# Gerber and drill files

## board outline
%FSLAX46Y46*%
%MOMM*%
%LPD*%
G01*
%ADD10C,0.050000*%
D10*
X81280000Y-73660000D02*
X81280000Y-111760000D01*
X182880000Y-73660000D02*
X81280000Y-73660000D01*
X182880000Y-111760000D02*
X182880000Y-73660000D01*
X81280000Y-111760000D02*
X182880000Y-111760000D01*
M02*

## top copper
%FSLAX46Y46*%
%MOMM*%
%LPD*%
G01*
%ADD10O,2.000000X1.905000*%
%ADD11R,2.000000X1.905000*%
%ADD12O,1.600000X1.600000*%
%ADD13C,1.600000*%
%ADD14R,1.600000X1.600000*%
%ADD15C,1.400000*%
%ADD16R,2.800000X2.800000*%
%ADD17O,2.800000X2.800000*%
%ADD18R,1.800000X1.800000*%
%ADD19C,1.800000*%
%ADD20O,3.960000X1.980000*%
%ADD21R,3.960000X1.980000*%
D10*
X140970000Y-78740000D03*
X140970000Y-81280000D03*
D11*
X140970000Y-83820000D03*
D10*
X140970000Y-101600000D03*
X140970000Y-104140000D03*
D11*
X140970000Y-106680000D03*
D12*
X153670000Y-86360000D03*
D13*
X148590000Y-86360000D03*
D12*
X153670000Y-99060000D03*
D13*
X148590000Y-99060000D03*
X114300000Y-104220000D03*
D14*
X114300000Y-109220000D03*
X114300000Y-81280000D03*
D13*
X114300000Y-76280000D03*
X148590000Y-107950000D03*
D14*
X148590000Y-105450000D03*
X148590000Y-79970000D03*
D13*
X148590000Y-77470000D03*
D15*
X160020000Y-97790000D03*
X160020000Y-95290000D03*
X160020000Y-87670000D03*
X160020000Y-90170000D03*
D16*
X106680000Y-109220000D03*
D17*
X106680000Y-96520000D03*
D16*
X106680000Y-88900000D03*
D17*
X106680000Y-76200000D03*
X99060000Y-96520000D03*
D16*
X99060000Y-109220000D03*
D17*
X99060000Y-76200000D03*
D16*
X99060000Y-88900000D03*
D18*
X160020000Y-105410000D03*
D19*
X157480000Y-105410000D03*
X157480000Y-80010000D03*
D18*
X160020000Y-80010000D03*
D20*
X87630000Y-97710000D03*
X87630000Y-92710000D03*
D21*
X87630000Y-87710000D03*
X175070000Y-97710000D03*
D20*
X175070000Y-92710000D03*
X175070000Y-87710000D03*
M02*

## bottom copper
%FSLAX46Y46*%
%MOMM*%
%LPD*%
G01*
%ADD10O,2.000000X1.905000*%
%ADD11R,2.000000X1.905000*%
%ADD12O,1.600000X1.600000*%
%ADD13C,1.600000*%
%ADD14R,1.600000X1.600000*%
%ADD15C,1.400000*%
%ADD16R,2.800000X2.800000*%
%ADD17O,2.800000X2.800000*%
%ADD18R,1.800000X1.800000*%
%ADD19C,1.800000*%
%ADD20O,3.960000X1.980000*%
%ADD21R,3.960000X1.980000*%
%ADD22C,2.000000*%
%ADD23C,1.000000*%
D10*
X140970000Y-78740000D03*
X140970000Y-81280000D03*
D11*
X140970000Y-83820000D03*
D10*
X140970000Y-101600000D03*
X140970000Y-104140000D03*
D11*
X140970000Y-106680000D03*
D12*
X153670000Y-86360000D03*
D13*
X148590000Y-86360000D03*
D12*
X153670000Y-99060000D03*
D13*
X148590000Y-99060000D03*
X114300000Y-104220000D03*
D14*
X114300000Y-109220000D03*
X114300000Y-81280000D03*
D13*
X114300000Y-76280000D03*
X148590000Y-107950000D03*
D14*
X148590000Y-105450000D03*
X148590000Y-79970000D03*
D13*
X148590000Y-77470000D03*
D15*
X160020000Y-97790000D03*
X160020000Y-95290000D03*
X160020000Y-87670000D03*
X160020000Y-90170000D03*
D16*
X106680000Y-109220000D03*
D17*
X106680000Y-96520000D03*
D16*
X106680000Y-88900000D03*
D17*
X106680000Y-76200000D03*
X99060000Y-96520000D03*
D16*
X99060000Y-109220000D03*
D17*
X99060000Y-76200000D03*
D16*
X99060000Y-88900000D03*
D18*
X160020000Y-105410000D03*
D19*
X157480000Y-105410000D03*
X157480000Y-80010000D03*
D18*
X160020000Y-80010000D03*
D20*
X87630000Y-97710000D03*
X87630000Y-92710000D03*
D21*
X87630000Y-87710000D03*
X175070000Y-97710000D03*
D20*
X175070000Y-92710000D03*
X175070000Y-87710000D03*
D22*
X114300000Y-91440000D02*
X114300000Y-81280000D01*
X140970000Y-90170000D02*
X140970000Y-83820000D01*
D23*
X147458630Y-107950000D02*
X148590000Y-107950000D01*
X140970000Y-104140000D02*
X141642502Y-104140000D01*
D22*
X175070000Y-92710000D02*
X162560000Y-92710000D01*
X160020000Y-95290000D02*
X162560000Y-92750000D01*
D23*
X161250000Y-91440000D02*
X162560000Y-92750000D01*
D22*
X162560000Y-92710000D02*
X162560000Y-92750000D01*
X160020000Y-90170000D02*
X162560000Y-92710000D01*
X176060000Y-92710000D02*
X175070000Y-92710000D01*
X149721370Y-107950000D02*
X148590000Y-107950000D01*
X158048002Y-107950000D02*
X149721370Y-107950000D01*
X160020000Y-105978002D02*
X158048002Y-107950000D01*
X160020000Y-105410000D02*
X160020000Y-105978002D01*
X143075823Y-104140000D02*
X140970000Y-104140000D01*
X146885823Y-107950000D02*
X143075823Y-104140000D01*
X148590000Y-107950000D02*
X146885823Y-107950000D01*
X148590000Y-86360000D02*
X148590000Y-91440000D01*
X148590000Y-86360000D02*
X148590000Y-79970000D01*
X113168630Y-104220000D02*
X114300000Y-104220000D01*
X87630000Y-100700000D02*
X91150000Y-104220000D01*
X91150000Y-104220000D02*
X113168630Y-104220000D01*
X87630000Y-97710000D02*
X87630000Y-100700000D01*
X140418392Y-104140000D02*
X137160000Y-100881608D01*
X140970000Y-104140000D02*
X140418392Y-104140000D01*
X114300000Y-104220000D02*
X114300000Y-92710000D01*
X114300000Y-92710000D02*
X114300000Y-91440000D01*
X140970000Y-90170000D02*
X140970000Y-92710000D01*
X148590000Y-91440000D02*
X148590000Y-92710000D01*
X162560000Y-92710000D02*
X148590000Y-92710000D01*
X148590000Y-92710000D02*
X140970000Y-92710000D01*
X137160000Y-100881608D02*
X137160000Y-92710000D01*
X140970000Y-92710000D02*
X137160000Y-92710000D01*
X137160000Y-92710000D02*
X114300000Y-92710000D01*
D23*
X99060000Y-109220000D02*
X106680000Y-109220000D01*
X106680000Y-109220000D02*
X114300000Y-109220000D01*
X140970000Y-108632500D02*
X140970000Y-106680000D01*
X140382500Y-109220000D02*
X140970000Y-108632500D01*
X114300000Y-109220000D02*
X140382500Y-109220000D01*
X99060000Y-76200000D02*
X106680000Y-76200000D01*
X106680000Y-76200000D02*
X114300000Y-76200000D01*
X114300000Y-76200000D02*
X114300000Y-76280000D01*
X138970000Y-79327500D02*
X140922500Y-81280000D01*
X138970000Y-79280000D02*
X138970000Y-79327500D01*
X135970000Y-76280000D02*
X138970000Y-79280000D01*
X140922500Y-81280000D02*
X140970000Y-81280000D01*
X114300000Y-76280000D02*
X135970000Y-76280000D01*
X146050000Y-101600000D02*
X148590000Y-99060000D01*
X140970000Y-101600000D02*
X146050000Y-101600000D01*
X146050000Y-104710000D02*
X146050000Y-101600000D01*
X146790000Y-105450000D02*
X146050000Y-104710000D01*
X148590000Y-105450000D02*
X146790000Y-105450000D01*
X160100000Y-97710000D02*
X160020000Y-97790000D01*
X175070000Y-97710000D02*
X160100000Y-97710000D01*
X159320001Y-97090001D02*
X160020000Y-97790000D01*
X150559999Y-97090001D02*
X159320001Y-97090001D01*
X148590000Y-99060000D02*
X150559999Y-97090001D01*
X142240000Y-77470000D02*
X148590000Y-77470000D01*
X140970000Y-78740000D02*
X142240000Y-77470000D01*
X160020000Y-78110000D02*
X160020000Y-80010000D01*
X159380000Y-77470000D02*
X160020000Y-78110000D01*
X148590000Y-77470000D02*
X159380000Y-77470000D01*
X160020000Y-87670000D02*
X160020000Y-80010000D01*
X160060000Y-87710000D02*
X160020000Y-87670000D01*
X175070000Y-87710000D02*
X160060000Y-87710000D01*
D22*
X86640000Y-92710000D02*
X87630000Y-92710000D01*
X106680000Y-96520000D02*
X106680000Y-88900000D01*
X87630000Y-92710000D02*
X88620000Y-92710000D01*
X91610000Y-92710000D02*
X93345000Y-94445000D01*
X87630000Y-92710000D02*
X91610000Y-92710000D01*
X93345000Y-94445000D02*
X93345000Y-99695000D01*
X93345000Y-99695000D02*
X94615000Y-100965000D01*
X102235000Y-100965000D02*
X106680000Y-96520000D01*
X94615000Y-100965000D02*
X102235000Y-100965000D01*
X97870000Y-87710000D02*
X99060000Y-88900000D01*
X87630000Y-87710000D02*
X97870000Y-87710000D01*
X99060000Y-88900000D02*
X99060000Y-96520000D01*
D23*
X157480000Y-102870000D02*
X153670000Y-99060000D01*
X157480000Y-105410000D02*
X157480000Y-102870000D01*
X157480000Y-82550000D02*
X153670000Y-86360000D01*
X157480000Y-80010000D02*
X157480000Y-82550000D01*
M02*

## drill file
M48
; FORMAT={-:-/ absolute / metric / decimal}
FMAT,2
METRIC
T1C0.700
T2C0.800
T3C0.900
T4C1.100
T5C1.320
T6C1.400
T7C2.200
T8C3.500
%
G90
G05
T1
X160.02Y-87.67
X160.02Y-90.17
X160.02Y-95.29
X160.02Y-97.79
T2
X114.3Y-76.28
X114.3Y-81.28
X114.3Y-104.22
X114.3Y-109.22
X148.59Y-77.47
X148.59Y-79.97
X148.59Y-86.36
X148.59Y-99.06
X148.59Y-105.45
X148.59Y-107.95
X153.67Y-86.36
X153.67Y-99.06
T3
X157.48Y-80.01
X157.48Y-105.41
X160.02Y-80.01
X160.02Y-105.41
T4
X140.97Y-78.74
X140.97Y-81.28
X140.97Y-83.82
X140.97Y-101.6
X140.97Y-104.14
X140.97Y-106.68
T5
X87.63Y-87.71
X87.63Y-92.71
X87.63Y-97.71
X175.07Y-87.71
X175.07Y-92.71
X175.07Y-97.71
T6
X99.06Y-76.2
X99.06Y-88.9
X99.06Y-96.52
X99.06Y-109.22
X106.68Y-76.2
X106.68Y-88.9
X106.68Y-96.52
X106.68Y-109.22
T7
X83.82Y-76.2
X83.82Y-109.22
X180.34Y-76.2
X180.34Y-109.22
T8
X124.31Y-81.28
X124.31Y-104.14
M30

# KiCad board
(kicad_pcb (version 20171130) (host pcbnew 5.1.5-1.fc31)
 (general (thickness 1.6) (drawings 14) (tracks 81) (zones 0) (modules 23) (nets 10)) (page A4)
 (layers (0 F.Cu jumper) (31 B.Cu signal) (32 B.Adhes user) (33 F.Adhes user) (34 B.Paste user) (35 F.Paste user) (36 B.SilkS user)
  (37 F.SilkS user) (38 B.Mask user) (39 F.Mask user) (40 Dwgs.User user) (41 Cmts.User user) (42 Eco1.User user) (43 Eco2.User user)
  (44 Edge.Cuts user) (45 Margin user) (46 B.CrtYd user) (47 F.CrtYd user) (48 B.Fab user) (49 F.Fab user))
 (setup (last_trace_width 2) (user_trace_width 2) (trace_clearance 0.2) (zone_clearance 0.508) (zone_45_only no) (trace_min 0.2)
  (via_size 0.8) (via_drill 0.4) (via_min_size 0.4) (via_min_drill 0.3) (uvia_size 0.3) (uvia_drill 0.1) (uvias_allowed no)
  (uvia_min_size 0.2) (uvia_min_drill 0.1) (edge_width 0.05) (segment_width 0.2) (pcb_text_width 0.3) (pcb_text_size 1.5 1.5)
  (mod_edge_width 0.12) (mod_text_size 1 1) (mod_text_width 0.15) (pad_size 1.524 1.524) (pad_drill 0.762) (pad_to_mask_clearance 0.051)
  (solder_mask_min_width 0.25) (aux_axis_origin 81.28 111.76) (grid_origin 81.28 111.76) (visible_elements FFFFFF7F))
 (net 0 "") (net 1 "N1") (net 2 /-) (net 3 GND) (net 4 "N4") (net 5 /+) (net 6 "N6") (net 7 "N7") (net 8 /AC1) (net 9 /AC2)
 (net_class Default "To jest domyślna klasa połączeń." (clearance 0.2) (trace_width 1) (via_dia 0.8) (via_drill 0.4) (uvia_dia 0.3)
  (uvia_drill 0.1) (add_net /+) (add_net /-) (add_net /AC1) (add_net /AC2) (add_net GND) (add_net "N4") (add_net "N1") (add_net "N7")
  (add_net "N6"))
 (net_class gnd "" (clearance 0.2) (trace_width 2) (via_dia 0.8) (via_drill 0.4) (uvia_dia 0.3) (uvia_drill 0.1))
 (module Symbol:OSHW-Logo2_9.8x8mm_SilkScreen (layer F.Cu) (at 114.3 87.63)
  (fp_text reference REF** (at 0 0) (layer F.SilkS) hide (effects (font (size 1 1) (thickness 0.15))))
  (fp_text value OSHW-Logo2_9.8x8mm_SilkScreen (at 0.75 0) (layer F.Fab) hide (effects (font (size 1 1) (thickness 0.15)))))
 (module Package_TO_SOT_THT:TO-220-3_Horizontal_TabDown (layer F.Cu) (at 140.97 83.82 90)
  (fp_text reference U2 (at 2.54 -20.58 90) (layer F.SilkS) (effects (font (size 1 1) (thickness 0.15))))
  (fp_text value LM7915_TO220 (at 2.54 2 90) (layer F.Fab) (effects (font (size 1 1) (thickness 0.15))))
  (pad 3 thru_hole oval (at 5.08 0 90) (size 1.905 2) (drill 1.1) (layers *.Cu *.Mask) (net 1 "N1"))
  (pad 2 thru_hole oval (at 2.54 0 90) (size 1.905 2) (drill 1.1) (layers *.Cu *.Mask) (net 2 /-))
  (pad 1 thru_hole rect (at 0 0 90) (size 1.905 2) (drill 1.1) (layers *.Cu *.Mask) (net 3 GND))
  (pad "" np_thru_hole oval (at 2.54 -16.66 90) (size 3.5 3.5) (drill 3.5) (layers *.Cu *.Mask)))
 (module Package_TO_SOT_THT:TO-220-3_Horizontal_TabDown (layer F.Cu) (at 140.97 106.68 90)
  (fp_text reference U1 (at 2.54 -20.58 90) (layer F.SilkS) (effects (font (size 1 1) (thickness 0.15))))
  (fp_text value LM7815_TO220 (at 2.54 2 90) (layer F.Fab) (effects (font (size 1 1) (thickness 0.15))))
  (pad 3 thru_hole oval (at 5.08 0 90) (size 1.905 2) (drill 1.1) (layers *.Cu *.Mask) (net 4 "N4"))
  (pad 2 thru_hole oval (at 2.54 0 90) (size 1.905 2) (drill 1.1) (layers *.Cu *.Mask) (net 3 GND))
  (pad 1 thru_hole rect (at 0 0 90) (size 1.905 2) (drill 1.1) (layers *.Cu *.Mask) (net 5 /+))
  (pad "" np_thru_hole oval (at 2.54 -16.66 90) (size 3.5 3.5) (drill 3.5) (layers *.Cu *.Mask)))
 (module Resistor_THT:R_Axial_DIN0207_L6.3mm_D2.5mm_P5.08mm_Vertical (layer F.Cu) (at 148.59 86.36)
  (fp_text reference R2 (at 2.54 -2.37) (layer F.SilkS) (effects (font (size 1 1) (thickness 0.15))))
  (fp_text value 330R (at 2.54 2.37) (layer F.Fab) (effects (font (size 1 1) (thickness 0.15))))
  (pad 2 thru_hole oval (at 5.08 0) (size 1.6 1.6) (drill 0.8) (layers *.Cu *.Mask) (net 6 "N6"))
  (pad 1 thru_hole circle (at 0 0) (size 1.6 1.6) (drill 0.8) (layers *.Cu *.Mask) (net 3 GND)))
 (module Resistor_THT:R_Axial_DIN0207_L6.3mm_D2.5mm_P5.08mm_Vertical (layer F.Cu) (at 148.59 99.06)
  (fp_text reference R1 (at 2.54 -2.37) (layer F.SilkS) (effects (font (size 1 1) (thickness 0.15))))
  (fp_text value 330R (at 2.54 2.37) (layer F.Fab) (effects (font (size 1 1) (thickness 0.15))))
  (pad 2 thru_hole oval (at 5.08 0) (size 1.6 1.6) (drill 0.8) (layers *.Cu *.Mask) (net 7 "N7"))
  (pad 1 thru_hole circle (at 0 0) (size 1.6 1.6) (drill 0.8) (layers *.Cu *.Mask) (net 4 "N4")))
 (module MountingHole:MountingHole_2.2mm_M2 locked (layer F.Cu) (at 83.82 109.22)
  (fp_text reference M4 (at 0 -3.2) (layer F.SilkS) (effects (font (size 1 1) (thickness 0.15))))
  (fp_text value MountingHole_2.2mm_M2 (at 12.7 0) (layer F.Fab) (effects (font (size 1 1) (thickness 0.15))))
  (pad 1 np_thru_hole circle (at 0 0) (size 2.2 2.2) (drill 2.2) (layers *.Cu *.Mask)))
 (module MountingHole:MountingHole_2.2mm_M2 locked (layer F.Cu) (at 180.34 109.22)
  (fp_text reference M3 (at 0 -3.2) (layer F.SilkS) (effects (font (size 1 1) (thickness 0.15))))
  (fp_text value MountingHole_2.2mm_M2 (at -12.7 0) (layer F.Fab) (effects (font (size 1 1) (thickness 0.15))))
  (pad 1 np_thru_hole circle (at 0 0) (size 2.2 2.2) (drill 2.2) (layers *.Cu *.Mask)))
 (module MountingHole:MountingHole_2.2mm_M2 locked (layer F.Cu) (at 180.34 76.2)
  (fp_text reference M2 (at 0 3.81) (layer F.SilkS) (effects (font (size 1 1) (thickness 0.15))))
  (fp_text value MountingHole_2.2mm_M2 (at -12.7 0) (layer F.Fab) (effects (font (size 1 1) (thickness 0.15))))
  (pad 1 np_thru_hole circle (at 0 0) (size 2.2 2.2) (drill 2.2) (layers *.Cu *.Mask)))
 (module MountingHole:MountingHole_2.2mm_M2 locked (layer F.Cu) (at 83.82 76.2)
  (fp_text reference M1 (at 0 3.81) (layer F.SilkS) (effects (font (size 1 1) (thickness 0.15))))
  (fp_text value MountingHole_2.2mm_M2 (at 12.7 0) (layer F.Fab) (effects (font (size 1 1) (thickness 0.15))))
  (pad 1 np_thru_hole circle (at 0 0) (size 2.2 2.2) (drill 2.2) (layers *.Cu *.Mask)))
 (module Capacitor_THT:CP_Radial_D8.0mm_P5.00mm (layer F.Cu) (at 114.3 109.22 90)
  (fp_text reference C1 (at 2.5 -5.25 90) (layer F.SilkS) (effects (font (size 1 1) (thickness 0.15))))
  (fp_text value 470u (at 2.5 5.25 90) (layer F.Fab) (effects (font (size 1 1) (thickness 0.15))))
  (pad 2 thru_hole circle (at 5 0 90) (size 1.6 1.6) (drill 0.8) (layers *.Cu *.Mask) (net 3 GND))
  (pad 1 thru_hole rect (at 0 0 90) (size 1.6 1.6) (drill 0.8) (layers *.Cu *.Mask) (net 5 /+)))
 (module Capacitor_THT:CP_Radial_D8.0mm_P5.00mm (layer F.Cu) (at 114.3 81.28 90)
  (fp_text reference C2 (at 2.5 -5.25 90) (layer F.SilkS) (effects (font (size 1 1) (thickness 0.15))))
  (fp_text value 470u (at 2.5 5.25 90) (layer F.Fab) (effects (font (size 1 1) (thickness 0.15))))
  (pad 1 thru_hole rect (at 0 0 90) (size 1.6 1.6) (drill 0.8) (layers *.Cu *.Mask) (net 3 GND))
  (pad 2 thru_hole circle (at 5 0 90) (size 1.6 1.6) (drill 0.8) (layers *.Cu *.Mask) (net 2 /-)))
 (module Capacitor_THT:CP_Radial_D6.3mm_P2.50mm (layer F.Cu) (at 148.59 105.45 270)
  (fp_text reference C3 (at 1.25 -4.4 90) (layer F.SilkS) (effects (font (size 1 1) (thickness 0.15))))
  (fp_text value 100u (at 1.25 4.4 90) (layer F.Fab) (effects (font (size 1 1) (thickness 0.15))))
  (pad 2 thru_hole circle (at 2.5 0 270) (size 1.6 1.6) (drill 0.8) (layers *.Cu *.Mask) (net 3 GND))
  (pad 1 thru_hole rect (at 0 0 270) (size 1.6 1.6) (drill 0.8) (layers *.Cu *.Mask) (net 4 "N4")))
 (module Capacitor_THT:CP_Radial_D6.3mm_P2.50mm (layer F.Cu) (at 148.59 79.97 90)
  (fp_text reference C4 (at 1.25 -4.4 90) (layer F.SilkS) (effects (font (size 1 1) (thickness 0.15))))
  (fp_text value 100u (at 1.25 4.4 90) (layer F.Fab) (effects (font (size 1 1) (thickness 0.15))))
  (pad 1 thru_hole rect (at 0 0 90) (size 1.6 1.6) (drill 0.8) (layers *.Cu *.Mask) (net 3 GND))
  (pad 2 thru_hole circle (at 2.5 0 90) (size 1.6 1.6) (drill 0.8) (layers *.Cu *.Mask) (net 1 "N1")))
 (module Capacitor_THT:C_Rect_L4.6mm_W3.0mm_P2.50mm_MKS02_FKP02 (layer F.Cu) (at 160.02 97.79 90)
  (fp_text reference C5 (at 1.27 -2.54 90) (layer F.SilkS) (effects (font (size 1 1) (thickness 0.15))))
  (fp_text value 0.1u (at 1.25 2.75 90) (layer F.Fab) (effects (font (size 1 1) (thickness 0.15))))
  (pad 1 thru_hole circle (at 0 0 90) (size 1.4 1.4) (drill 0.7) (layers *.Cu *.Mask) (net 4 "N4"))
  (pad 2 thru_hole circle (at 2.5 0 90) (size 1.4 1.4) (drill 0.7) (layers *.Cu *.Mask) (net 3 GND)))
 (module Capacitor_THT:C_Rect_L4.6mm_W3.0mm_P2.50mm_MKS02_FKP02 (layer F.Cu) (at 160.02 90.17 90)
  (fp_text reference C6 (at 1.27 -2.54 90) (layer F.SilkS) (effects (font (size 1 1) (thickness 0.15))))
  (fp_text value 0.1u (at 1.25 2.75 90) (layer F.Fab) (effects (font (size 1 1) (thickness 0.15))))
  (pad 2 thru_hole circle (at 2.5 0 90) (size 1.4 1.4) (drill 0.7) (layers *.Cu *.Mask) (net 1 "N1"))
  (pad 1 thru_hole circle (at 0 0 90) (size 1.4 1.4) (drill 0.7) (layers *.Cu *.Mask) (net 3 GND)))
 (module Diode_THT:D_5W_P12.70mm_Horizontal (layer F.Cu) (at 106.68 109.22 90)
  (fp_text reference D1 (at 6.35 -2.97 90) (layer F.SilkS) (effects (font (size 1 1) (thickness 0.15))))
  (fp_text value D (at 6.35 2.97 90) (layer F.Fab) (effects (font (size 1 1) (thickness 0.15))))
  (pad 1 thru_hole rect (at 0 0 90) (size 2.8 2.8) (drill 1.4) (layers *.Cu *.Mask) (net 5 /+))
  (pad 2 thru_hole oval (at 12.7 0 90) (size 2.8 2.8) (drill 1.4) (layers *.Cu *.Mask) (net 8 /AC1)))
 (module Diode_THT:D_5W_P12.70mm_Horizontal (layer F.Cu) (at 106.68 88.9 90)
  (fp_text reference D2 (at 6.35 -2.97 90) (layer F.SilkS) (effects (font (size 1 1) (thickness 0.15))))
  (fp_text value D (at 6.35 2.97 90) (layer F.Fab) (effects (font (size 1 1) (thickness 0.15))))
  (pad 1 thru_hole rect (at 0 0 90) (size 2.8 2.8) (drill 1.4) (layers *.Cu *.Mask) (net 8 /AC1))
  (pad 2 thru_hole oval (at 12.7 0 90) (size 2.8 2.8) (drill 1.4) (layers *.Cu *.Mask) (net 2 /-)))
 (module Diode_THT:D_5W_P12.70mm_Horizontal (layer F.Cu) (at 99.06 109.22 90)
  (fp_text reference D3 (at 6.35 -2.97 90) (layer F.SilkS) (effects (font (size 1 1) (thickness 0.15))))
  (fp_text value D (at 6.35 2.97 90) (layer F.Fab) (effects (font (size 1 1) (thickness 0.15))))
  (pad 2 thru_hole oval (at 12.7 0 90) (size 2.8 2.8) (drill 1.4) (layers *.Cu *.Mask) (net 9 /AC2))
  (pad 1 thru_hole rect (at 0 0 90) (size 2.8 2.8) (drill 1.4) (layers *.Cu *.Mask) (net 5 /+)))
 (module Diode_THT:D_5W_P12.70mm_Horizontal (layer F.Cu) (at 99.06 88.9 90)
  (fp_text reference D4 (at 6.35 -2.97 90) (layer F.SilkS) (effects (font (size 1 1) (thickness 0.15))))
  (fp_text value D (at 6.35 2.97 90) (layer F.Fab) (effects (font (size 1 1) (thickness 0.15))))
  (pad 2 thru_hole oval (at 12.7 0 90) (size 2.8 2.8) (drill 1.4) (layers *.Cu *.Mask) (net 2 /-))
  (pad 1 thru_hole rect (at 0 0 90) (size 2.8 2.8) (drill 1.4) (layers *.Cu *.Mask) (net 9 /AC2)))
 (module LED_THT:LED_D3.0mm (layer F.Cu) (at 160.02 105.41 180)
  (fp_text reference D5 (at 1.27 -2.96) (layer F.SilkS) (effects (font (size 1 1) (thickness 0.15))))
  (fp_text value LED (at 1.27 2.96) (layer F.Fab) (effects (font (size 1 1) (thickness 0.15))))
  (pad 1 thru_hole rect (at 0 0 180) (size 1.8 1.8) (drill 0.9) (layers *.Cu *.Mask) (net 3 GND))
  (pad 2 thru_hole circle (at 2.54 0 180) (size 1.8 1.8) (drill 0.9) (layers *.Cu *.Mask) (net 7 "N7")))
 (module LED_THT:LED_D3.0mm (layer F.Cu) (at 160.02 80.01 180)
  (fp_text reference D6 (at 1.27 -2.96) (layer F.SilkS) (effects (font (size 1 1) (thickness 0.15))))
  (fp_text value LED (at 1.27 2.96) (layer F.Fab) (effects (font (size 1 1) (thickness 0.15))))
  (pad 2 thru_hole circle (at 2.54 0 180) (size 1.8 1.8) (drill 0.9) (layers *.Cu *.Mask) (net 6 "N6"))
  (pad 1 thru_hole rect (at 0 0 180) (size 1.8 1.8) (drill 0.9) (layers *.Cu *.Mask) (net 1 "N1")))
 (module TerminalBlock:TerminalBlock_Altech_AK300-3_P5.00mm (layer F.Cu) (at 87.63 87.71 270)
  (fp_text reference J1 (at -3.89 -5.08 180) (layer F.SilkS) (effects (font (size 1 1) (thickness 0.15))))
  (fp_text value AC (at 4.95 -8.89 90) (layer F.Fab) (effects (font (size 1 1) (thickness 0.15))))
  (pad 3 thru_hole oval (at 10 0 270) (size 1.98 3.96) (drill 1.32) (layers *.Cu *.Mask) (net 3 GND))
  (pad 2 thru_hole oval (at 5 0 270) (size 1.98 3.96) (drill 1.32) (layers *.Cu *.Mask) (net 8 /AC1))
  (pad 1 thru_hole rect (at 0 0 270) (size 1.98 3.96) (drill 1.32) (layers *.Cu *.Mask) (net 9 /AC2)))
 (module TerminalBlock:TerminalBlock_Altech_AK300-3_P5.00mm (layer F.Cu) (at 175.07 97.71 90)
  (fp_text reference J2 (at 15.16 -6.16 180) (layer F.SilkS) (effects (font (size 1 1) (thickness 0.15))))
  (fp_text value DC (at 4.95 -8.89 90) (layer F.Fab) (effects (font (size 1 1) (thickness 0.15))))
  (pad 1 thru_hole rect (at 0 0 90) (size 1.98 3.96) (drill 1.32) (layers *.Cu *.Mask) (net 4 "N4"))
  (pad 2 thru_hole oval (at 5 0 90) (size 1.98 3.96) (drill 1.32) (layers *.Cu *.Mask) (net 3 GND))
  (pad 3 thru_hole oval (at 10 0 90) (size 1.98 3.96) (drill 1.32) (layers *.Cu *.Mask) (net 1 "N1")))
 (gr_line (start 81.28 73.66) (end 81.28 111.76) (layer Edge.Cuts) (width 0.05))
 (gr_line (start 182.88 73.66) (end 81.28 73.66) (layer Edge.Cuts) (width 0.05))
 (gr_line (start 182.88 111.76) (end 182.88 73.66) (layer Edge.Cuts) (width 0.05))
 (gr_line (start 81.28 111.76) (end 182.88 111.76) (layer Edge.Cuts) (width 0.05))
 (segment (start 114.3 91.44) (end 114.3 81.28) (width 2) (layer B.Cu) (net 3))
 (segment (start 140.97 90.17) (end 140.97 83.82) (width 2) (layer B.Cu) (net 3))
 (segment (start 147.45863 107.95) (end 148.59 107.95) (width 1) (layer B.Cu) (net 3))
 (segment (start 140.97 104.14) (end 141.642502 104.14) (width 1) (layer B.Cu) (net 3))
 (segment (start 175.07 92.71) (end 162.56 92.71) (width 2) (layer B.Cu) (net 3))
 (segment (start 160.02 95.29) (end 162.56 92.75) (width 2) (layer B.Cu) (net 3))
 (segment (start 161.25 91.44) (end 162.56 92.75) (width 1) (layer B.Cu) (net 3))
 (segment (start 162.56 92.71) (end 162.56 92.75) (width 2) (layer B.Cu) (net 3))
 (segment (start 160.02 90.17) (end 162.56 92.71) (width 2) (layer B.Cu) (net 3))
 (segment (start 176.06 92.71) (end 175.07 92.71) (width 2) (layer B.Cu) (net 3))
 (segment (start 149.72137 107.95) (end 148.59 107.95) (width 2) (layer B.Cu) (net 3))
 (segment (start 158.048002 107.95) (end 149.72137 107.95) (width 2) (layer B.Cu) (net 3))
 (segment (start 160.02 105.978002) (end 158.048002 107.95) (width 2) (layer B.Cu) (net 3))
 (segment (start 160.02 105.41) (end 160.02 105.978002) (width 2) (layer B.Cu) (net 3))
 (segment (start 143.075823 104.14) (end 140.97 104.14) (width 2) (layer B.Cu) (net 3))
 (segment (start 146.885823 107.95) (end 143.075823 104.14) (width 2) (layer B.Cu) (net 3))
 (segment (start 148.59 107.95) (end 146.885823 107.95) (width 2) (layer B.Cu) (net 3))
 (segment (start 148.59 86.36) (end 148.59 91.44) (width 2) (layer B.Cu) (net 3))
 (segment (start 148.59 86.36) (end 148.59 79.97) (width 2) (layer B.Cu) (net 3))
 (segment (start 113.16863 104.22) (end 114.3 104.22) (width 2) (layer B.Cu) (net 3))
 (segment (start 87.63 100.7) (end 91.15 104.22) (width 2) (layer B.Cu) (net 3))
 (segment (start 91.15 104.22) (end 113.16863 104.22) (width 2) (layer B.Cu) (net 3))
 (segment (start 87.63 97.71) (end 87.63 100.7) (width 2) (layer B.Cu) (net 3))
 (segment (start 140.418392 104.14) (end 137.16 100.881608) (width 2) (layer B.Cu) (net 3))
 (segment (start 140.97 104.14) (end 140.418392 104.14) (width 2) (layer B.Cu) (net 3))
 (segment (start 114.3 104.22) (end 114.3 92.71) (width 2) (layer B.Cu) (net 3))
 (segment (start 114.3 92.71) (end 114.3 91.44) (width 2) (layer B.Cu) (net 3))
 (segment (start 140.97 90.17) (end 140.97 92.71) (width 2) (layer B.Cu) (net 3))
 (segment (start 148.59 91.44) (end 148.59 92.71) (width 2) (layer B.Cu) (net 3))
 (segment (start 162.56 92.71) (end 148.59 92.71) (width 2) (layer B.Cu) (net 3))
 (segment (start 148.59 92.71) (end 140.97 92.71) (width 2) (layer B.Cu) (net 3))
 (segment (start 137.16 100.881608) (end 137.16 92.71) (width 2) (layer B.Cu) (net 3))
 (segment (start 140.97 92.71) (end 137.16 92.71) (width 2) (layer B.Cu) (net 3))
 (segment (start 137.16 92.71) (end 114.3 92.71) (width 2) (layer B.Cu) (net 3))
 (segment (start 99.06 109.22) (end 106.68 109.22) (width 1) (layer B.Cu) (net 5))
 (segment (start 106.68 109.22) (end 114.3 109.22) (width 1) (layer B.Cu) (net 5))
 (segment (start 140.97 108.6325) (end 140.97 106.68) (width 1) (layer B.Cu) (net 5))
 (segment (start 140.3825 109.22) (end 140.97 108.6325) (width 1) (layer B.Cu) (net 5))
 (segment (start 114.3 109.22) (end 140.3825 109.22) (width 1) (layer B.Cu) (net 5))
 (segment (start 99.06 76.2) (end 106.68 76.2) (width 1) (layer B.Cu) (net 2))
 (segment (start 106.68 76.2) (end 114.3 76.2) (width 1) (layer B.Cu) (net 2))
 (segment (start 114.3 76.2) (end 114.3 76.28) (width 1) (layer B.Cu) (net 2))
 (segment (start 138.97 79.3275) (end 140.9225 81.28) (width 1) (layer B.Cu) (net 2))
 (segment (start 138.97 79.28) (end 138.97 79.3275) (width 1) (layer B.Cu) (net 2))
 (segment (start 135.97 76.28) (end 138.97 79.28) (width 1) (layer B.Cu) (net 2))
 (segment (start 140.9225 81.28) (end 140.97 81.28) (width 1) (layer B.Cu) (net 2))
 (segment (start 114.3 76.28) (end 135.97 76.28) (width 1) (layer B.Cu) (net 2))
 (segment (start 146.05 101.6) (end 148.59 99.06) (width 1) (layer B.Cu) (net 4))
 (segment (start 140.97 101.6) (end 146.05 101.6) (width 1) (layer B.Cu) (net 4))
 (segment (start 146.05 104.71) (end 146.05 101.6) (width 1) (layer B.Cu) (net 4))
 (segment (start 146.79 105.45) (end 146.05 104.71) (width 1) (layer B.Cu) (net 4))
 (segment (start 148.59 105.45) (end 146.79 105.45) (width 1) (layer B.Cu) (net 4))
 (segment (start 160.1 97.71) (end 160.02 97.79) (width 1) (layer B.Cu) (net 4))
 (segment (start 175.07 97.71) (end 160.1 97.71) (width 1) (layer B.Cu) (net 4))
 (segment (start 159.320001 97.090001) (end 160.02 97.79) (width 1) (layer B.Cu) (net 4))
 (segment (start 150.559999 97.090001) (end 159.320001 97.090001) (width 1) (layer B.Cu) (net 4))
 (segment (start 148.59 99.06) (end 150.559999 97.090001) (width 1) (layer B.Cu) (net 4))
 (segment (start 142.24 77.47) (end 148.59 77.47) (width 1) (layer B.Cu) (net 1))
 (segment (start 140.97 78.74) (end 142.24 77.47) (width 1) (layer B.Cu) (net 1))
 (segment (start 160.02 78.11) (end 160.02 80.01) (width 1) (layer B.Cu) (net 1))
 (segment (start 159.38 77.47) (end 160.02 78.11) (width 1) (layer B.Cu) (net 1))
 (segment (start 148.59 77.47) (end 159.38 77.47) (width 1) (layer B.Cu) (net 1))
 (segment (start 160.02 87.67) (end 160.02 80.01) (width 1) (layer B.Cu) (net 1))
 (segment (start 160.06 87.71) (end 160.02 87.67) (width 1) (layer B.Cu) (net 1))
 (segment (start 175.07 87.71) (end 160.06 87.71) (width 1) (layer B.Cu) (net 1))
 (segment (start 86.64 92.71) (end 87.63 92.71) (width 2) (layer B.Cu) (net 8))
 (segment (start 106.68 96.52) (end 106.68 88.9) (width 2) (layer B.Cu) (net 8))
 (segment (start 87.63 92.71) (end 88.62 92.71) (width 2) (layer B.Cu) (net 8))
 (segment (start 91.61 92.71) (end 93.345 94.445) (width 2) (layer B.Cu) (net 8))
 (segment (start 87.63 92.71) (end 91.61 92.71) (width 2) (layer B.Cu) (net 8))
 (segment (start 93.345 94.445) (end 93.345 99.695) (width 2) (layer B.Cu) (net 8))
 (segment (start 93.345 99.695) (end 94.615 100.965) (width 2) (layer B.Cu) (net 8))
 (segment (start 102.235 100.965) (end 106.68 96.52) (width 2) (layer B.Cu) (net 8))
 (segment (start 94.615 100.965) (end 102.235 100.965) (width 2) (layer B.Cu) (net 8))
 (segment (start 97.87 87.71) (end 99.06 88.9) (width 2) (layer B.Cu) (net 9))
 (segment (start 87.63 87.71) (end 97.87 87.71) (width 2) (layer B.Cu) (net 9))
 (segment (start 99.06 88.9) (end 99.06 96.52) (width 2) (layer B.Cu) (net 9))
 (segment (start 157.48 102.87) (end 153.67 99.06) (width 1) (layer B.Cu) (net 7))
 (segment (start 157.48 105.41) (end 157.48 102.87) (width 1) (layer B.Cu) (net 7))
 (segment (start 157.48 82.55) (end 153.67 86.36) (width 1) (layer B.Cu) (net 6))
 (segment (start 157.48 80.01) (end 157.48 82.55) (width 1) (layer B.Cu) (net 6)))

